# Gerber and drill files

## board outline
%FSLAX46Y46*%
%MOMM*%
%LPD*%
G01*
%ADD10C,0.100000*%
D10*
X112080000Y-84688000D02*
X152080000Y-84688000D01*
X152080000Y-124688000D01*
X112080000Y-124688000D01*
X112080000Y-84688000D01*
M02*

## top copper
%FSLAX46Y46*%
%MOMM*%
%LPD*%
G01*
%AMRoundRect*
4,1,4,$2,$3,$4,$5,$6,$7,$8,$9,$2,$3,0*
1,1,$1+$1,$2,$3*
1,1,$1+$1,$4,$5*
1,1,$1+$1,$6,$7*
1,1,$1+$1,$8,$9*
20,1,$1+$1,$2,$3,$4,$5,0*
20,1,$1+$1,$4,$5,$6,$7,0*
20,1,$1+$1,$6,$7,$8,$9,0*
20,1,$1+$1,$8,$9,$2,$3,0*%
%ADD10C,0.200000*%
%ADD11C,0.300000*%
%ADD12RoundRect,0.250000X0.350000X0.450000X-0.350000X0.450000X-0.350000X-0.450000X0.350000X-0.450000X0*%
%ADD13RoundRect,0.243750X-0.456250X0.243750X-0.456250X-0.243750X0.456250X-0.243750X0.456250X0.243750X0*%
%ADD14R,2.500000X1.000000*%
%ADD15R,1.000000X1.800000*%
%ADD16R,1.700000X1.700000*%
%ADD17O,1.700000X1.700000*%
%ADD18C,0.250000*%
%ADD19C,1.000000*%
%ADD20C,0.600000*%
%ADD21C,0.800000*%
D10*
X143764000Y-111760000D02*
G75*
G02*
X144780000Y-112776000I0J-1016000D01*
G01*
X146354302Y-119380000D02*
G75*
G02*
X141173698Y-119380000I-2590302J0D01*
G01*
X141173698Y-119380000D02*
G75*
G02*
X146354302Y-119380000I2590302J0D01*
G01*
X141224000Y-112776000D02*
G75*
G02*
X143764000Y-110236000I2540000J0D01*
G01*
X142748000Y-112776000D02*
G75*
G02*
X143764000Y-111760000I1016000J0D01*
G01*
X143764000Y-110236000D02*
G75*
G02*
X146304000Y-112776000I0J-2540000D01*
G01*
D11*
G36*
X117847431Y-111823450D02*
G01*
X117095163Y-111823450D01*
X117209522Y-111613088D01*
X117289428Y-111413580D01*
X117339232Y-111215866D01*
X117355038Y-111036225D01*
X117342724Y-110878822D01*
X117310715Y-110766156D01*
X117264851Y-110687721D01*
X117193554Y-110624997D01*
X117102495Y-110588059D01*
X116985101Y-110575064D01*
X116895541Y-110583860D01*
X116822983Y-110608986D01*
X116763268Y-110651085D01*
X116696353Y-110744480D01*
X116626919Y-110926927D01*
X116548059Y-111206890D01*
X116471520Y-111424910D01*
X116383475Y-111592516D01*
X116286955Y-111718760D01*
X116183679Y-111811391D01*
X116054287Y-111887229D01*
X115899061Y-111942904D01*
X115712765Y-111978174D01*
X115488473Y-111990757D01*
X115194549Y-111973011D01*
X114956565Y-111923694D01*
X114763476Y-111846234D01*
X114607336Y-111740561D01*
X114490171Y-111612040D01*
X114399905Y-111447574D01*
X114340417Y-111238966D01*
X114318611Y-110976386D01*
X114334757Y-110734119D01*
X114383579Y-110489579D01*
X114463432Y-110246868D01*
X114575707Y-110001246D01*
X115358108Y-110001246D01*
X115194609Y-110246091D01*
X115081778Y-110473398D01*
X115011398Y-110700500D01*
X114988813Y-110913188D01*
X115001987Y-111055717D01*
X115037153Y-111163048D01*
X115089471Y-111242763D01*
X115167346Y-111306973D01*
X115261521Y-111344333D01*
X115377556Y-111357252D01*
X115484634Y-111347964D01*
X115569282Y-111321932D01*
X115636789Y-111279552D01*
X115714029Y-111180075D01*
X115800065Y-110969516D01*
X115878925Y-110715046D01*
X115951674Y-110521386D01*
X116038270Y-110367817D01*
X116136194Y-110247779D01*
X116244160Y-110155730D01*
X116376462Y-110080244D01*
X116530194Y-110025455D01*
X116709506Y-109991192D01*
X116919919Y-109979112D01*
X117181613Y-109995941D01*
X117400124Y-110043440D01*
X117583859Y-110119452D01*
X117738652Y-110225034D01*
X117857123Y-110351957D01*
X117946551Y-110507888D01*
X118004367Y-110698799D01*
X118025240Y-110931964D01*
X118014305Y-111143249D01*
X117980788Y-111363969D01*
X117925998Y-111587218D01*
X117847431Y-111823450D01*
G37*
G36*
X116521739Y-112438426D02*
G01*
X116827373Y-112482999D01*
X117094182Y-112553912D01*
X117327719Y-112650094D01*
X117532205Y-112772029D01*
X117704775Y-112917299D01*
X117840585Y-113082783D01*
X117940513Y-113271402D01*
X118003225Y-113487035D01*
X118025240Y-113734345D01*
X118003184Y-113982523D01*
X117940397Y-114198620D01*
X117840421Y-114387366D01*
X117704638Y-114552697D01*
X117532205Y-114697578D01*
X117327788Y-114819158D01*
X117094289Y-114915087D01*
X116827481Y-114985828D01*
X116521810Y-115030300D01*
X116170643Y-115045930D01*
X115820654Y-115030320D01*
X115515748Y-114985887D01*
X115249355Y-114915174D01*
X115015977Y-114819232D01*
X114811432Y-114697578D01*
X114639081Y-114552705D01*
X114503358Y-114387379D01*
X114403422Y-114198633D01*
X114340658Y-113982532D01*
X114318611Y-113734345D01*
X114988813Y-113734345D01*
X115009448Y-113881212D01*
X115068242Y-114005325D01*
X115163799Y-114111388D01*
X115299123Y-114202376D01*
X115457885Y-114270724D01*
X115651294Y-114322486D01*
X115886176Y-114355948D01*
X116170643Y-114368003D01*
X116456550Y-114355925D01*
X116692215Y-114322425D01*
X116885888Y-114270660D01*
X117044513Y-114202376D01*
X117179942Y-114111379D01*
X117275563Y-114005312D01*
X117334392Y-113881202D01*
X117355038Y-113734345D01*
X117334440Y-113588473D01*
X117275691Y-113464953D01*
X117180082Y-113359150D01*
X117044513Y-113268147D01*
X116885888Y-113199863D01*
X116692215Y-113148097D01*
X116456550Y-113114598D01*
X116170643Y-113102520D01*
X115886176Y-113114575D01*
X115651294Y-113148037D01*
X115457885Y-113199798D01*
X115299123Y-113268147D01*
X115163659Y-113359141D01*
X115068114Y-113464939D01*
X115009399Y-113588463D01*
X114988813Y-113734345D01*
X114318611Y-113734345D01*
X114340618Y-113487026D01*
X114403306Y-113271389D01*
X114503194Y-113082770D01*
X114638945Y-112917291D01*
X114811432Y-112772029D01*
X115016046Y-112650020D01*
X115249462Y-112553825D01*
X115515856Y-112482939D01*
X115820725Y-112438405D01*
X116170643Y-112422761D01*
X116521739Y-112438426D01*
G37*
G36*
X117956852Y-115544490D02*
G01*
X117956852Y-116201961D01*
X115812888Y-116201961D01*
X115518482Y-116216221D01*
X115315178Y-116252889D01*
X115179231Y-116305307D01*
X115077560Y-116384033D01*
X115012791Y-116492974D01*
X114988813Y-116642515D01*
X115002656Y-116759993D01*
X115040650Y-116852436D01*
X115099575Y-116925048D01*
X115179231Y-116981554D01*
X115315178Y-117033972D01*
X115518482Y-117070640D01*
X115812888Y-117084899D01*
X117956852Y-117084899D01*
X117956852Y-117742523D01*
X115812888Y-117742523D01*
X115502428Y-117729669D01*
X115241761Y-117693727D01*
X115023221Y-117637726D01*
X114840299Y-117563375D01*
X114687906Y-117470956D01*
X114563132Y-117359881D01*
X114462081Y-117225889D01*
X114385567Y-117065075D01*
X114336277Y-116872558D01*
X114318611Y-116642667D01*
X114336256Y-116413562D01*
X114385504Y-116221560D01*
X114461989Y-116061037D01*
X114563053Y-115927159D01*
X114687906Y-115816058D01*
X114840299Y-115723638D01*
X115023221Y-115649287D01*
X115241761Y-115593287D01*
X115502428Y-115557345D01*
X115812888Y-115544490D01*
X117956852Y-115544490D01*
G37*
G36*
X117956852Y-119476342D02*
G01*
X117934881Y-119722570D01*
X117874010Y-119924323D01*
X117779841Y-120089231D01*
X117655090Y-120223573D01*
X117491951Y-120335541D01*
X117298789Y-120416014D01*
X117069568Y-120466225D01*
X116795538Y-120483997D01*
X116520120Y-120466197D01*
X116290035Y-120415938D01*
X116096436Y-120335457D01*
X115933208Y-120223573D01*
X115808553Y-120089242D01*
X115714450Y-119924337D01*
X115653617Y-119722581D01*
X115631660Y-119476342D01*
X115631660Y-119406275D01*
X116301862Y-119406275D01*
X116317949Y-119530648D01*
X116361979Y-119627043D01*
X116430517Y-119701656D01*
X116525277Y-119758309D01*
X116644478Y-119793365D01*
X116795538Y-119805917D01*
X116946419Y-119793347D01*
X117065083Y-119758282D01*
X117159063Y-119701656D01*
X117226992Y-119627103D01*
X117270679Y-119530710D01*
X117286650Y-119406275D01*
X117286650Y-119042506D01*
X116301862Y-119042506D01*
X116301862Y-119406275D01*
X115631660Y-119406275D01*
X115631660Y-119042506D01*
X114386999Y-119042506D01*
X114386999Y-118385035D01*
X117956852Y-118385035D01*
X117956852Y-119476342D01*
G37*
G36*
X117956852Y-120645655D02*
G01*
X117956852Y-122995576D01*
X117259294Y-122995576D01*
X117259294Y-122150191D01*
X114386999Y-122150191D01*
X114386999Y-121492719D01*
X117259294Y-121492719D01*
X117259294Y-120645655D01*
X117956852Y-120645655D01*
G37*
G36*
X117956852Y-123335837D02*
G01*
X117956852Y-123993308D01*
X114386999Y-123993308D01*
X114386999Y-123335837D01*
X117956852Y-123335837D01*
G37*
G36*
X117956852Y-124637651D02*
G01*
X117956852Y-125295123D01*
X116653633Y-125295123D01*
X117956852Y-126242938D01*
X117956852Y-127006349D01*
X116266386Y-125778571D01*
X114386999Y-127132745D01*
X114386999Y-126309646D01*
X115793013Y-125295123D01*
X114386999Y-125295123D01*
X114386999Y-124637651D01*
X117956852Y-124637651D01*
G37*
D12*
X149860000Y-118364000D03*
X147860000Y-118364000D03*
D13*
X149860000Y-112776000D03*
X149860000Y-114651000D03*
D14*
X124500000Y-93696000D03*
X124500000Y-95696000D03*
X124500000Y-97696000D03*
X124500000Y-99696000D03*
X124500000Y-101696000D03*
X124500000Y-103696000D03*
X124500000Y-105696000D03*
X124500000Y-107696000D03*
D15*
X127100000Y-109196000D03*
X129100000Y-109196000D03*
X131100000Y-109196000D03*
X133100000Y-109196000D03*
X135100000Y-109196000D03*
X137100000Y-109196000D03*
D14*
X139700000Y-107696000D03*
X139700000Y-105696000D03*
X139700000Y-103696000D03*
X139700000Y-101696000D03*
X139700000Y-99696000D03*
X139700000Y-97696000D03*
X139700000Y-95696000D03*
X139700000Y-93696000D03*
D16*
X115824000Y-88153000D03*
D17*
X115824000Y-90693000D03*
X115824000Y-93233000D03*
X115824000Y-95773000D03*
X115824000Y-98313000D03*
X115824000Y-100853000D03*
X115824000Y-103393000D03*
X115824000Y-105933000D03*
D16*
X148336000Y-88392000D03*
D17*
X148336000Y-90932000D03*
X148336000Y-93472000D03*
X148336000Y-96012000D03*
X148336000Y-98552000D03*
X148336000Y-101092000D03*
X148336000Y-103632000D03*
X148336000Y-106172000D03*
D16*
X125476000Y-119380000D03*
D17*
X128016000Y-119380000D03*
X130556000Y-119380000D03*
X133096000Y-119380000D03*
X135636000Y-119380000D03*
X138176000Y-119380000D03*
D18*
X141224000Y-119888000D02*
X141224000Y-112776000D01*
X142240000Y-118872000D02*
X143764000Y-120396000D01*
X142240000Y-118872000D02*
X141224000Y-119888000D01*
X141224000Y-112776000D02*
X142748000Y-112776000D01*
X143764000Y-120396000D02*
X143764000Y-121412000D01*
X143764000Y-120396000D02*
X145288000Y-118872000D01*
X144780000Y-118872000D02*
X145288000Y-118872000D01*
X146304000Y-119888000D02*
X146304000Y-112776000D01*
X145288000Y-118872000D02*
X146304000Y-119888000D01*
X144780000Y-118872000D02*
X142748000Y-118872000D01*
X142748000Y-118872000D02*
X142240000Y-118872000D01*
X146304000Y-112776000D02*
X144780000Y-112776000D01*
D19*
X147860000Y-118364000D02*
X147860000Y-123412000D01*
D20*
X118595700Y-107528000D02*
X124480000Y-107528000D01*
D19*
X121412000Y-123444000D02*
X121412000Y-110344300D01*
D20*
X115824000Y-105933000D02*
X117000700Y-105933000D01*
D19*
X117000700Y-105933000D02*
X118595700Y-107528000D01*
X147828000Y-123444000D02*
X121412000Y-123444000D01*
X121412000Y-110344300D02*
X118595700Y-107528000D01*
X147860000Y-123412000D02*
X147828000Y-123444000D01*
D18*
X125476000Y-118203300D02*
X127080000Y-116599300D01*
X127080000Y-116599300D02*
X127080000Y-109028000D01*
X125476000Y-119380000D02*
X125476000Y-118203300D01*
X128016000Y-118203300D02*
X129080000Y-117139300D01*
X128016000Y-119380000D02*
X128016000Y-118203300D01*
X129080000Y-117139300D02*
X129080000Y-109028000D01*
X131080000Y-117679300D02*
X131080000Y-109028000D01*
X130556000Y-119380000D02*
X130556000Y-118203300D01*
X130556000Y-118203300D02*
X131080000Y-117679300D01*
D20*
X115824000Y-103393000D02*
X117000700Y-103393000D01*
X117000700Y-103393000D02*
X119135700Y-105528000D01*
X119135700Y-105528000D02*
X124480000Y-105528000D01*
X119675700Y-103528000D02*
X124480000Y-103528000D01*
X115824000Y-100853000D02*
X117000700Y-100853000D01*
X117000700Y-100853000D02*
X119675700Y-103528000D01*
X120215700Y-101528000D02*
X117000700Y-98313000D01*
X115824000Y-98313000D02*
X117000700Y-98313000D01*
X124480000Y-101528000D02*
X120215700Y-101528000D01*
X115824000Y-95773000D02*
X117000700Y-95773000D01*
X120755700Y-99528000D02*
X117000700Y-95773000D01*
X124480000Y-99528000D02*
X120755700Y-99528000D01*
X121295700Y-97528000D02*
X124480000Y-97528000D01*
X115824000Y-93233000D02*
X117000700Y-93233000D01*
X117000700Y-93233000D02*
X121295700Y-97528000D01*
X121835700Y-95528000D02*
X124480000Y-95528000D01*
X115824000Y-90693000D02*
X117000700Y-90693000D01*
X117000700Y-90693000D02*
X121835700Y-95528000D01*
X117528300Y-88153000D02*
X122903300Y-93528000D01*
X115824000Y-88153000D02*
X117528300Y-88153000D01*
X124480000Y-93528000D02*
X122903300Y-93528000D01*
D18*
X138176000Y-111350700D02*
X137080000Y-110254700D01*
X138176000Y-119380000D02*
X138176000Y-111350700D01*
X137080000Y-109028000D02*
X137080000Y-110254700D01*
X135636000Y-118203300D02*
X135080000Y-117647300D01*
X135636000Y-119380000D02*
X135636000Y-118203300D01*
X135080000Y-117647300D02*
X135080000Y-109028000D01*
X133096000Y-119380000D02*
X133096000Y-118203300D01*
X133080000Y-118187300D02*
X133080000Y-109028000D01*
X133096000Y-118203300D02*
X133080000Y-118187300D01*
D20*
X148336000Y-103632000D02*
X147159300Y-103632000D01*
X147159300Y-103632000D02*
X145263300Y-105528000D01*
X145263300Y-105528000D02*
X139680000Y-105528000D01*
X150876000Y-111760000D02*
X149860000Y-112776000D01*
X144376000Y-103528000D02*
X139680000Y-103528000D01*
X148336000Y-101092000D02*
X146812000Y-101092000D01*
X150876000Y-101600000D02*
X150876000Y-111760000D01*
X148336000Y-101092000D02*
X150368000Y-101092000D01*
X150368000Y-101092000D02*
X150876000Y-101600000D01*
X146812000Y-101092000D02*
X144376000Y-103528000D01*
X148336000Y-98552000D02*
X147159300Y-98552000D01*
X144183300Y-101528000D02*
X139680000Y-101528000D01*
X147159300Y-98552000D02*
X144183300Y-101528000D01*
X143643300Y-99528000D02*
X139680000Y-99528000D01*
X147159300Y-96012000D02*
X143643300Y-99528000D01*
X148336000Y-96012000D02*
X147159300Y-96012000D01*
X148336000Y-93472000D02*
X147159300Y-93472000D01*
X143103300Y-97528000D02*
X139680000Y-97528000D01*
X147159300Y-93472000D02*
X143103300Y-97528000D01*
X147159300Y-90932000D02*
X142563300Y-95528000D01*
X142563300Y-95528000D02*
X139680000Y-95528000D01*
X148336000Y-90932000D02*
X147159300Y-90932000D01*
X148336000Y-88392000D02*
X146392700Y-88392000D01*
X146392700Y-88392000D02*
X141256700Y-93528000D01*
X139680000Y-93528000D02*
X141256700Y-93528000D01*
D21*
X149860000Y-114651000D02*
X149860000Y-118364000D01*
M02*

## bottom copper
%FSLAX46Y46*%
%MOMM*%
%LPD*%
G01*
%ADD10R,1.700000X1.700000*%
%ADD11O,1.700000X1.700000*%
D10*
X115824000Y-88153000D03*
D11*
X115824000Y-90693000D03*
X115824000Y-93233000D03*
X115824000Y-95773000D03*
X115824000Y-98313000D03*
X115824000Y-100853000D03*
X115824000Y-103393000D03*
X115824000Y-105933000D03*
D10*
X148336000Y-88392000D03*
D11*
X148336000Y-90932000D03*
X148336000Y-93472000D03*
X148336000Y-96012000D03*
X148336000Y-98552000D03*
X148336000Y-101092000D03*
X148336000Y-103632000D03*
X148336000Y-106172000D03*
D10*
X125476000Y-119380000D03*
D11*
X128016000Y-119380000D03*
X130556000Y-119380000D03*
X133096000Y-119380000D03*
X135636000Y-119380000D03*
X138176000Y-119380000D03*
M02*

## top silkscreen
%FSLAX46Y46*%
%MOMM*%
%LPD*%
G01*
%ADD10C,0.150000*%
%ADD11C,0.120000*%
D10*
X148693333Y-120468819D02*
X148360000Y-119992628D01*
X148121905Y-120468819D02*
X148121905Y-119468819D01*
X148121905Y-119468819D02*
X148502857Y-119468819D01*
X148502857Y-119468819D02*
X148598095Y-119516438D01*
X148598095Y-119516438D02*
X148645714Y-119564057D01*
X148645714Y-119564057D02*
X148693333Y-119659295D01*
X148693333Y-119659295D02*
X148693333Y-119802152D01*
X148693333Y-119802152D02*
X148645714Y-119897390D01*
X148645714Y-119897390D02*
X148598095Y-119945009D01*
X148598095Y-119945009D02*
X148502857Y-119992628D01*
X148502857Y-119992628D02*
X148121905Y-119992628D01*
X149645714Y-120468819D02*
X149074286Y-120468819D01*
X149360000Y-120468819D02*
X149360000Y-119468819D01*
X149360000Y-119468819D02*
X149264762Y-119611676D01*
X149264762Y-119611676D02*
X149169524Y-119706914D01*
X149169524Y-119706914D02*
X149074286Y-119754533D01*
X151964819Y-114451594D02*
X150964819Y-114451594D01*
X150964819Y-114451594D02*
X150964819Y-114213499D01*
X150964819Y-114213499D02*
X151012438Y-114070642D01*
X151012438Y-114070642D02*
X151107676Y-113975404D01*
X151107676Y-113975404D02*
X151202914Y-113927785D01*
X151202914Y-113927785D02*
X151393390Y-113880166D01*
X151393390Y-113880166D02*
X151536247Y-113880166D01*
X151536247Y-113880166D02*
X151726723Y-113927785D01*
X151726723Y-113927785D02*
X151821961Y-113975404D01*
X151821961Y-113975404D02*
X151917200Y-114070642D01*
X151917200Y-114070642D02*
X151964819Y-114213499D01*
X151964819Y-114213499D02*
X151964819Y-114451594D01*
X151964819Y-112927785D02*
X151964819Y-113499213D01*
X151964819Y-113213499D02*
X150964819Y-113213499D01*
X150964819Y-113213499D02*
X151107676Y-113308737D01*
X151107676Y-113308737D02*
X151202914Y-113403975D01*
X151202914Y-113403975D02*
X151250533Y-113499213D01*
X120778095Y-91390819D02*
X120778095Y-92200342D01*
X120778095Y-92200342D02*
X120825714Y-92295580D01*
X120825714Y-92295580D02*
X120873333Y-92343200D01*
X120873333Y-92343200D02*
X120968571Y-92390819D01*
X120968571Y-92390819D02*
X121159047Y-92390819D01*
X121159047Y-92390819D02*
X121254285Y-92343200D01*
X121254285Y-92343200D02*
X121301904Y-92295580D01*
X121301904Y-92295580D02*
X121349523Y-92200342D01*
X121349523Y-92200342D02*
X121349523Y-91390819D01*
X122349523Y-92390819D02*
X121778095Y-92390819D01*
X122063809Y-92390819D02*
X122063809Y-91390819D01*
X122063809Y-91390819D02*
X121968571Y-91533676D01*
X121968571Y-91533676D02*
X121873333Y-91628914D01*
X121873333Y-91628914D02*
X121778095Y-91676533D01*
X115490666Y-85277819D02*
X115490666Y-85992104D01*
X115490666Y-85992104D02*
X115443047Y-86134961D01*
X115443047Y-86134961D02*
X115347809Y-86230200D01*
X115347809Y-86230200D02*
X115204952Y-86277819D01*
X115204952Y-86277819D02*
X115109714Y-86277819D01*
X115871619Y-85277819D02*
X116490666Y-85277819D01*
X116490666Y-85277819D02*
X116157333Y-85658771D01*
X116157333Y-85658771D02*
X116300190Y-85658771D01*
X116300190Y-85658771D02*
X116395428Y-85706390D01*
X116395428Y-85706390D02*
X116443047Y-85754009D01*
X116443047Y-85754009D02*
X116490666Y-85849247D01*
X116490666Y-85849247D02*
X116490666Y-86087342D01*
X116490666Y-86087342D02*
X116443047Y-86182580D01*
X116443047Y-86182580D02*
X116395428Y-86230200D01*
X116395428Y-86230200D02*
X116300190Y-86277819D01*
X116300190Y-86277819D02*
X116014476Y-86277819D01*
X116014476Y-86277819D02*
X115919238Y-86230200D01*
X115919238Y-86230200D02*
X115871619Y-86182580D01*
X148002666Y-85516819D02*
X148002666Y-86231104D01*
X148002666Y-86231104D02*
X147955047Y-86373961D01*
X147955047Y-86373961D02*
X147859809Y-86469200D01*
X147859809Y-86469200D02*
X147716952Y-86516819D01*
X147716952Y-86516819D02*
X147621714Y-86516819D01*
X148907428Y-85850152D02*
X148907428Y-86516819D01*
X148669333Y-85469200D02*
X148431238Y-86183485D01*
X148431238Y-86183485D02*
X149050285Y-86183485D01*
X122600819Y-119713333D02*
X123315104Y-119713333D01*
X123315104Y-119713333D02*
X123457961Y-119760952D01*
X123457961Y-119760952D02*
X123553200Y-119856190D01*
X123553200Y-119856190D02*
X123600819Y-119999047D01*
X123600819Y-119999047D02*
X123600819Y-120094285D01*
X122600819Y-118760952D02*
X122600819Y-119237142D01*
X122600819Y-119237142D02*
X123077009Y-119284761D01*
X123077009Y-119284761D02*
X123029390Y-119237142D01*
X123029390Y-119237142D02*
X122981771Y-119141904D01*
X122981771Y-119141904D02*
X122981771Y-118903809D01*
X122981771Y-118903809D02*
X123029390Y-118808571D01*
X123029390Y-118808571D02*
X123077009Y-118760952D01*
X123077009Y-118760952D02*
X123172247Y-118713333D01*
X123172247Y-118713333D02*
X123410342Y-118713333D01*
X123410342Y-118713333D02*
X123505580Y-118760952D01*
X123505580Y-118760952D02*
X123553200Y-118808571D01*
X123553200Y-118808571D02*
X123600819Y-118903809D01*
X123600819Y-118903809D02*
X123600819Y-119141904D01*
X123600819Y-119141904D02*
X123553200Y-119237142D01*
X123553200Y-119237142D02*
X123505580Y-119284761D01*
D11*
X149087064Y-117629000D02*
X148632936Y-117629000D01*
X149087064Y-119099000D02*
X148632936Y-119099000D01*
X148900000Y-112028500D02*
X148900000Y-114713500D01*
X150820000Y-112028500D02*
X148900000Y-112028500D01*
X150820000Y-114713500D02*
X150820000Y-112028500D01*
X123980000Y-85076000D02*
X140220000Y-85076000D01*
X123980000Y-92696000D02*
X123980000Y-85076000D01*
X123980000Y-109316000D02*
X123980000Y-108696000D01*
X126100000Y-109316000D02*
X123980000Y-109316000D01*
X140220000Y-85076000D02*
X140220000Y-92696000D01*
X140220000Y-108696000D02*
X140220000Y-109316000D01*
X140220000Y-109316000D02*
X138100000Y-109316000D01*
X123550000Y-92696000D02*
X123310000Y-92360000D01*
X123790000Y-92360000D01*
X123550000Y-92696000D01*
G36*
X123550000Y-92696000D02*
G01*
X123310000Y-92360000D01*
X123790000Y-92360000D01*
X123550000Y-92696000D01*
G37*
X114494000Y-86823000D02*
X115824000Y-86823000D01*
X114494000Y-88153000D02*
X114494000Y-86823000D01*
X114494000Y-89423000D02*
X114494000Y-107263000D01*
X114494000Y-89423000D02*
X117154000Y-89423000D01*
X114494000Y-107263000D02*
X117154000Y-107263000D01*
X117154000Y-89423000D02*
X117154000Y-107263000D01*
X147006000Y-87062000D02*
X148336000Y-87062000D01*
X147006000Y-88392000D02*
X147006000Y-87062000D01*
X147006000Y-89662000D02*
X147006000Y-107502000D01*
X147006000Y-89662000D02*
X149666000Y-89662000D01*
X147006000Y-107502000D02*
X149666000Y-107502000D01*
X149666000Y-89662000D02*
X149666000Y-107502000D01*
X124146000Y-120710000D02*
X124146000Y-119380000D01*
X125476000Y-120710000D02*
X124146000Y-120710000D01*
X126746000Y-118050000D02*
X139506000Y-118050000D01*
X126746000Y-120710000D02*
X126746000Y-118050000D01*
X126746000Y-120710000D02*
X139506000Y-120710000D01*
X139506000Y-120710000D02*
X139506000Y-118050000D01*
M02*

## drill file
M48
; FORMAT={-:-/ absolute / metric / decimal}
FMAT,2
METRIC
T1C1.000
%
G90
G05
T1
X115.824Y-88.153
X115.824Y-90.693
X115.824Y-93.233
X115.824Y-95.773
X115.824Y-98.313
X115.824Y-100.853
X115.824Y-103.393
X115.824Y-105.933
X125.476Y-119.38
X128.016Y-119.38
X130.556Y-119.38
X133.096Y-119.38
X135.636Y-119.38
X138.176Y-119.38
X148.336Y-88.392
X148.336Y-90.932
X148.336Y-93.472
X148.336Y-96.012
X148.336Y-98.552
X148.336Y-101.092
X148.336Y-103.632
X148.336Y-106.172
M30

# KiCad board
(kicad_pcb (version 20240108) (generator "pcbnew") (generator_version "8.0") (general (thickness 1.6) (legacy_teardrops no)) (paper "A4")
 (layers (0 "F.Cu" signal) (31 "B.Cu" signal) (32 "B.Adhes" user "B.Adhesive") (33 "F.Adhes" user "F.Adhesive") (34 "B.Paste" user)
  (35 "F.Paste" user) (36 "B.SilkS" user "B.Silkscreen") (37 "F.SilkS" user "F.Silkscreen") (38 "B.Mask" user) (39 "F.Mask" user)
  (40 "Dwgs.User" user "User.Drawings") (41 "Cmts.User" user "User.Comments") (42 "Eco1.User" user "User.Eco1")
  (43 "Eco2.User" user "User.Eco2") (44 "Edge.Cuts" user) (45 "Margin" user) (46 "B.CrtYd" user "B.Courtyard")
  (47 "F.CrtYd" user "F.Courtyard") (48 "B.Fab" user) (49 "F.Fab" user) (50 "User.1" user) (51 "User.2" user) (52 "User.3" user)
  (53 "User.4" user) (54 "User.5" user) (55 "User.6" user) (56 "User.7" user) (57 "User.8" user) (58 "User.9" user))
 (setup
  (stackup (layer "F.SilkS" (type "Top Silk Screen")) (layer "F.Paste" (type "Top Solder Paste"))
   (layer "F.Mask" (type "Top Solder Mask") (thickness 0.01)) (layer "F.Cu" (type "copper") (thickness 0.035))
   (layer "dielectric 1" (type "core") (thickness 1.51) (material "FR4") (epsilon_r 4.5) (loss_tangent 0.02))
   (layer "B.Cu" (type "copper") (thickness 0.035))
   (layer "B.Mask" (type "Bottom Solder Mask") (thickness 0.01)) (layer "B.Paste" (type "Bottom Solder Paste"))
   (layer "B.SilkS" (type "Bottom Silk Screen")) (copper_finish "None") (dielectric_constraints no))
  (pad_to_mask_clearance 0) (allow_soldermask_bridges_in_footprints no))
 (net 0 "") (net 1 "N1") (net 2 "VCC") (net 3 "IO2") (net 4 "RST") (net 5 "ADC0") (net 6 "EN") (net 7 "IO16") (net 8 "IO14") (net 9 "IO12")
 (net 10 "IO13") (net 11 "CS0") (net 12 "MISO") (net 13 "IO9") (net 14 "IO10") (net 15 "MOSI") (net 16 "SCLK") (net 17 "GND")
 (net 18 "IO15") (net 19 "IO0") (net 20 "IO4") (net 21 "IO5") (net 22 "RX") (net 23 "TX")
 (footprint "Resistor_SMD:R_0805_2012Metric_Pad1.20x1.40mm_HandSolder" (layer "F.Cu") (at 148.86 118.364 180)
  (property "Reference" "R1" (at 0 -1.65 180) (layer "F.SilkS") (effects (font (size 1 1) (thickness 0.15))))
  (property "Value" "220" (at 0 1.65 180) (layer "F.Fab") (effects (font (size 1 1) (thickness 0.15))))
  (fp_line (start -0.227064 0.735) (end 0.227064 0.735) (stroke (width 0.12) (type solid)) (layer "F.SilkS"))
  (fp_line (start -0.227064 -0.735) (end 0.227064 -0.735) (stroke (width 0.12) (type solid)) (layer "F.SilkS"))
  (pad "1" smd roundrect (at -1 0 180) (size 1.2 1.4) (layers "F.Cu" "F.Paste" "F.Mask") (roundrect_rratio 0.208333) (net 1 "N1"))
  (pad "2" smd roundrect (at 1 0 180) (size 1.2 1.4) (layers "F.Cu" "F.Paste" "F.Mask") (roundrect_rratio 0.208333) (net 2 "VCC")))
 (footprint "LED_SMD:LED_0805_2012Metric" (layer "F.Cu") (at 149.86 113.7135 -90)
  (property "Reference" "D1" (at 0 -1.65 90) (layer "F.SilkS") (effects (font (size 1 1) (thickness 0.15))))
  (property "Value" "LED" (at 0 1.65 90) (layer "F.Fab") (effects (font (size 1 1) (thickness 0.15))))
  (fp_line (start -1.685 0.96) (end 1 0.96) (stroke (width 0.12) (type solid)) (layer "F.SilkS"))
  (fp_line (start -1.685 -0.96) (end -1.685 0.96) (stroke (width 0.12) (type solid)) (layer "F.SilkS"))
  (fp_line (start 1 -0.96) (end -1.685 -0.96) (stroke (width 0.12) (type solid)) (layer "F.SilkS"))
  (pad "1" smd roundrect (at -0.9375 0 270) (size 0.975 1.4) (layers "F.Cu" "F.Paste" "F.Mask") (roundrect_rratio 0.25) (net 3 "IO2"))
  (pad "2" smd roundrect (at 0.9375 0 270) (size 0.975 1.4) (layers "F.Cu" "F.Paste" "F.Mask") (roundrect_rratio 0.25) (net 1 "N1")))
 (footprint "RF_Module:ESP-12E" (layer "F.Cu") (at 132.1 97.196)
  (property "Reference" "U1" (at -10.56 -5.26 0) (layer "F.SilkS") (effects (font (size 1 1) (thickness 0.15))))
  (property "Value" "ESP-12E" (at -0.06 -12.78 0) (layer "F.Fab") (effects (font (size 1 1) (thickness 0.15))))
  (fp_line (start -8.12 -12.12) (end 8.12 -12.12) (stroke (width 0.12) (type solid)) (layer "F.SilkS"))
  (fp_line (start -8.12 -4.5) (end -8.12 -12.12) (stroke (width 0.12) (type solid)) (layer "F.SilkS"))
  (fp_line (start -8.12 12.12) (end -8.12 11.5) (stroke (width 0.12) (type solid)) (layer "F.SilkS"))
  (fp_line (start -6 12.12) (end -8.12 12.12) (stroke (width 0.12) (type solid)) (layer "F.SilkS"))
  (fp_line (start 8.12 -12.12) (end 8.12 -4.5) (stroke (width 0.12) (type solid)) (layer "F.SilkS"))
  (fp_line (start 8.12 11.5) (end 8.12 12.12) (stroke (width 0.12) (type solid)) (layer "F.SilkS"))
  (fp_line (start 8.12 12.12) (end 6 12.12) (stroke (width 0.12) (type solid)) (layer "F.SilkS"))
  (fp_poly
   (pts (xy -8.55 -4.5) (xy -8.79 -4.836) (xy -8.31 -4.836) (xy -8.55 -4.5)) (stroke (width 0.12) (type solid)) (fill solid)
   (layer "F.SilkS"))
  (pad "1" smd rect (at -7.6 -3.5) (size 2.5 1) (layers "F.Cu" "F.Paste" "F.Mask") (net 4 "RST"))
  (pad "2" smd rect (at -7.6 -1.5) (size 2.5 1) (layers "F.Cu" "F.Paste" "F.Mask") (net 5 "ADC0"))
  (pad "3" smd rect (at -7.6 0.5) (size 2.5 1) (layers "F.Cu" "F.Paste" "F.Mask") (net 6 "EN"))
  (pad "4" smd rect (at -7.6 2.5) (size 2.5 1) (layers "F.Cu" "F.Paste" "F.Mask") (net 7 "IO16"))
  (pad "5" smd rect (at -7.6 4.5) (size 2.5 1) (layers "F.Cu" "F.Paste" "F.Mask") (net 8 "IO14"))
  (pad "6" smd rect (at -7.6 6.5) (size 2.5 1) (layers "F.Cu" "F.Paste" "F.Mask") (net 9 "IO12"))
  (pad "7" smd rect (at -7.6 8.5) (size 2.5 1) (layers "F.Cu" "F.Paste" "F.Mask") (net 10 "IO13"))
  (pad "8" smd rect (at -7.6 10.5) (size 2.5 1) (layers "F.Cu" "F.Paste" "F.Mask") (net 2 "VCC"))
  (pad "9" smd rect (at -5 12) (size 1 1.8) (layers "F.Cu" "F.Paste" "F.Mask") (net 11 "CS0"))
  (pad "10" smd rect (at -3 12) (size 1 1.8) (layers "F.Cu" "F.Paste" "F.Mask") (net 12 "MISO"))
  (pad "11" smd rect (at -1 12) (size 1 1.8) (layers "F.Cu" "F.Paste" "F.Mask") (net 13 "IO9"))
  (pad "12" smd rect (at 1 12) (size 1 1.8) (layers "F.Cu" "F.Paste" "F.Mask") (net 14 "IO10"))
  (pad "13" smd rect (at 3 12) (size 1 1.8) (layers "F.Cu" "F.Paste" "F.Mask") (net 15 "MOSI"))
  (pad "14" smd rect (at 5 12) (size 1 1.8) (layers "F.Cu" "F.Paste" "F.Mask") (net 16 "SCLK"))
  (pad "15" smd rect (at 7.6 10.5) (size 2.5 1) (layers "F.Cu" "F.Paste" "F.Mask") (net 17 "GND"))
  (pad "16" smd rect (at 7.6 8.5) (size 2.5 1) (layers "F.Cu" "F.Paste" "F.Mask") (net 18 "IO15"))
  (pad "17" smd rect (at 7.6 6.5) (size 2.5 1) (layers "F.Cu" "F.Paste" "F.Mask") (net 3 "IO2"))
  (pad "18" smd rect (at 7.6 4.5) (size 2.5 1) (layers "F.Cu" "F.Paste" "F.Mask") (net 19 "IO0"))
  (pad "19" smd rect (at 7.6 2.5) (size 2.5 1) (layers "F.Cu" "F.Paste" "F.Mask") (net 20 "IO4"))
  (pad "20" smd rect (at 7.6 0.5) (size 2.5 1) (layers "F.Cu" "F.Paste" "F.Mask") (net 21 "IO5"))
  (pad "21" smd rect (at 7.6 -1.5) (size 2.5 1) (layers "F.Cu" "F.Paste" "F.Mask") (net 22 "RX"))
  (pad "22" smd rect (at 7.6 -3.5) (size 2.5 1) (layers "F.Cu" "F.Paste" "F.Mask") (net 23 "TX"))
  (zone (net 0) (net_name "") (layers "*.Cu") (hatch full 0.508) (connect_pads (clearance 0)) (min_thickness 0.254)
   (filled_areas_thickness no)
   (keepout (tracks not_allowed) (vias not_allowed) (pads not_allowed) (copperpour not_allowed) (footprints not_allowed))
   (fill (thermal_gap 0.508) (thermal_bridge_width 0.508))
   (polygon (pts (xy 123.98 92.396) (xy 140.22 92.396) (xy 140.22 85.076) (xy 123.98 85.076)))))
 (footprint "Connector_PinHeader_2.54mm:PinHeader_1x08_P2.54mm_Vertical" (layer "F.Cu") (at 115.824 88.153)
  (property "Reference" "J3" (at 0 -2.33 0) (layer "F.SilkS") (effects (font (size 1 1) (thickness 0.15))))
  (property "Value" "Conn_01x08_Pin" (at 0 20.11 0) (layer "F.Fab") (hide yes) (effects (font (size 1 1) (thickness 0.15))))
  (fp_line (start -1.33 -1.33) (end 0 -1.33) (stroke (width 0.12) (type solid)) (layer "F.SilkS"))
  (fp_line (start -1.33 0) (end -1.33 -1.33) (stroke (width 0.12) (type solid)) (layer "F.SilkS"))
  (fp_line (start -1.33 1.27) (end -1.33 19.11) (stroke (width 0.12) (type solid)) (layer "F.SilkS"))
  (fp_line (start -1.33 1.27) (end 1.33 1.27) (stroke (width 0.12) (type solid)) (layer "F.SilkS"))
  (fp_line (start -1.33 19.11) (end 1.33 19.11) (stroke (width 0.12) (type solid)) (layer "F.SilkS"))
  (fp_line (start 1.33 1.27) (end 1.33 19.11) (stroke (width 0.12) (type solid)) (layer "F.SilkS"))
  (pad "1" thru_hole rect (at 0 0) (size 1.7 1.7) (drill 1) (layers "*.Cu" "*.Mask") (remove_unused_layers no) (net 4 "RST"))
  (pad "2" thru_hole oval (at 0 2.54) (size 1.7 1.7) (drill 1) (layers "*.Cu" "*.Mask") (remove_unused_layers no) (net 5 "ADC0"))
  (pad "3" thru_hole oval (at 0 5.08) (size 1.7 1.7) (drill 1) (layers "*.Cu" "*.Mask") (remove_unused_layers no) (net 6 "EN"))
  (pad "4" thru_hole oval (at 0 7.62) (size 1.7 1.7) (drill 1) (layers "*.Cu" "*.Mask") (remove_unused_layers no) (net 7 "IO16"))
  (pad "5" thru_hole oval (at 0 10.16) (size 1.7 1.7) (drill 1) (layers "*.Cu" "*.Mask") (remove_unused_layers no) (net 8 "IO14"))
  (pad "6" thru_hole oval (at 0 12.7) (size 1.7 1.7) (drill 1) (layers "*.Cu" "*.Mask") (remove_unused_layers no) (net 9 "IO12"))
  (pad "7" thru_hole oval (at 0 15.24) (size 1.7 1.7) (drill 1) (layers "*.Cu" "*.Mask") (remove_unused_layers no) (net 10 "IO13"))
  (pad "8" thru_hole oval (at 0 17.78) (size 1.7 1.7) (drill 1) (layers "*.Cu" "*.Mask") (remove_unused_layers no) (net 2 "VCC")))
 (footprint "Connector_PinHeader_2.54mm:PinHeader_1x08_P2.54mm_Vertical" (layer "F.Cu") (at 148.336 88.392)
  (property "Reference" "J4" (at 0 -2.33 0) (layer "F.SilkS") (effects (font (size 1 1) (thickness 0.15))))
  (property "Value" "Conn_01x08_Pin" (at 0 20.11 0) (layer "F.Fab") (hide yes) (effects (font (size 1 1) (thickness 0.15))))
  (fp_line (start -1.33 -1.33) (end 0 -1.33) (stroke (width 0.12) (type solid)) (layer "F.SilkS"))
  (fp_line (start -1.33 0) (end -1.33 -1.33) (stroke (width 0.12) (type solid)) (layer "F.SilkS"))
  (fp_line (start -1.33 1.27) (end -1.33 19.11) (stroke (width 0.12) (type solid)) (layer "F.SilkS"))
  (fp_line (start -1.33 1.27) (end 1.33 1.27) (stroke (width 0.12) (type solid)) (layer "F.SilkS"))
  (fp_line (start -1.33 19.11) (end 1.33 19.11) (stroke (width 0.12) (type solid)) (layer "F.SilkS"))
  (fp_line (start 1.33 1.27) (end 1.33 19.11) (stroke (width 0.12) (type solid)) (layer "F.SilkS"))
  (pad "1" thru_hole rect (at 0 0) (size 1.7 1.7) (drill 1) (layers "*.Cu" "*.Mask") (remove_unused_layers no) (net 23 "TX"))
  (pad "2" thru_hole oval (at 0 2.54) (size 1.7 1.7) (drill 1) (layers "*.Cu" "*.Mask") (remove_unused_layers no) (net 22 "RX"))
  (pad "3" thru_hole oval (at 0 5.08) (size 1.7 1.7) (drill 1) (layers "*.Cu" "*.Mask") (remove_unused_layers no) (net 21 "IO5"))
  (pad "4" thru_hole oval (at 0 7.62) (size 1.7 1.7) (drill 1) (layers "*.Cu" "*.Mask") (remove_unused_layers no) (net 20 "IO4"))
  (pad "5" thru_hole oval (at 0 10.16) (size 1.7 1.7) (drill 1) (layers "*.Cu" "*.Mask") (remove_unused_layers no) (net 19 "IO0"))
  (pad "6" thru_hole oval (at 0 12.7) (size 1.7 1.7) (drill 1) (layers "*.Cu" "*.Mask") (remove_unused_layers no) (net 3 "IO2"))
  (pad "7" thru_hole oval (at 0 15.24) (size 1.7 1.7) (drill 1) (layers "*.Cu" "*.Mask") (remove_unused_layers no) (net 18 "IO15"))
  (pad "8" thru_hole oval (at 0 17.78) (size 1.7 1.7) (drill 1) (layers "*.Cu" "*.Mask") (remove_unused_layers no) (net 17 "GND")))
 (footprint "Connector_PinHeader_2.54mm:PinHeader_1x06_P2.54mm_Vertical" (layer "F.Cu") (at 125.476 119.38 90)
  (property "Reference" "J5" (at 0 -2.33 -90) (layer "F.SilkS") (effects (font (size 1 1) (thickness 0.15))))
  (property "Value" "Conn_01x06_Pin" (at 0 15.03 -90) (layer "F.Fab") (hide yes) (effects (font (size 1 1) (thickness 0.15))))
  (fp_line (start -1.33 -1.33) (end 0 -1.33) (stroke (width 0.12) (type solid)) (layer "F.SilkS"))
  (fp_line (start -1.33 0) (end -1.33 -1.33) (stroke (width 0.12) (type solid)) (layer "F.SilkS"))
  (fp_line (start 1.33 1.27) (end 1.33 14.03) (stroke (width 0.12) (type solid)) (layer "F.SilkS"))
  (fp_line (start -1.33 1.27) (end 1.33 1.27) (stroke (width 0.12) (type solid)) (layer "F.SilkS"))
  (fp_line (start -1.33 1.27) (end -1.33 14.03) (stroke (width 0.12) (type solid)) (layer "F.SilkS"))
  (fp_line (start -1.33 14.03) (end 1.33 14.03) (stroke (width 0.12) (type solid)) (layer "F.SilkS"))
  (pad "1" thru_hole rect (at 0 0 90) (size 1.7 1.7) (drill 1) (layers "*.Cu" "*.Mask") (remove_unused_layers no) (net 11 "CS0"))
  (pad "2" thru_hole oval (at 0 2.54 90) (size 1.7 1.7) (drill 1) (layers "*.Cu" "*.Mask") (remove_unused_layers no) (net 12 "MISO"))
  (pad "3" thru_hole oval (at 0 5.08 90) (size 1.7 1.7) (drill 1) (layers "*.Cu" "*.Mask") (remove_unused_layers no) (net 13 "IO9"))
  (pad "4" thru_hole oval (at 0 7.62 90) (size 1.7 1.7) (drill 1) (layers "*.Cu" "*.Mask") (remove_unused_layers no) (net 14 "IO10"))
  (pad "5" thru_hole oval (at 0 10.16 90) (size 1.7 1.7) (drill 1) (layers "*.Cu" "*.Mask") (remove_unused_layers no) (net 15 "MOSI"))
  (pad "6" thru_hole oval (at 0 12.7 90) (size 1.7 1.7) (drill 1) (layers "*.Cu" "*.Mask") (remove_unused_layers no) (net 16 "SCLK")))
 (gr_arc (start 143.764 111.76) (mid 144.48242 112.05758) (end 144.78 112.776) (stroke (width 0.2) (type default)) (layer "F.Cu"))
 (gr_circle (center 143.764 119.38) (end 143.256 121.92) (stroke (width 0.2) (type default)) (fill none) (layer "F.Cu"))
 (gr_arc (start 141.224 112.776) (mid 141.967949 110.979949) (end 143.764 110.236) (stroke (width 0.2) (type default)) (layer "F.Cu"))
 (gr_arc (start 142.748 112.776) (mid 143.04558 112.05758) (end 143.764 111.76) (stroke (width 0.2) (type default)) (layer "F.Cu"))
 (gr_arc (start 143.764 110.236) (mid 145.560051 110.979949) (end 146.304 112.776) (stroke (width 0.2) (type default)) (layer "F.Cu"))
 (gr_rect (start 112.08 84.688) (end 152.08 124.688) (stroke (width 0.1) (type default)) (fill none) (layer "Edge.Cuts"))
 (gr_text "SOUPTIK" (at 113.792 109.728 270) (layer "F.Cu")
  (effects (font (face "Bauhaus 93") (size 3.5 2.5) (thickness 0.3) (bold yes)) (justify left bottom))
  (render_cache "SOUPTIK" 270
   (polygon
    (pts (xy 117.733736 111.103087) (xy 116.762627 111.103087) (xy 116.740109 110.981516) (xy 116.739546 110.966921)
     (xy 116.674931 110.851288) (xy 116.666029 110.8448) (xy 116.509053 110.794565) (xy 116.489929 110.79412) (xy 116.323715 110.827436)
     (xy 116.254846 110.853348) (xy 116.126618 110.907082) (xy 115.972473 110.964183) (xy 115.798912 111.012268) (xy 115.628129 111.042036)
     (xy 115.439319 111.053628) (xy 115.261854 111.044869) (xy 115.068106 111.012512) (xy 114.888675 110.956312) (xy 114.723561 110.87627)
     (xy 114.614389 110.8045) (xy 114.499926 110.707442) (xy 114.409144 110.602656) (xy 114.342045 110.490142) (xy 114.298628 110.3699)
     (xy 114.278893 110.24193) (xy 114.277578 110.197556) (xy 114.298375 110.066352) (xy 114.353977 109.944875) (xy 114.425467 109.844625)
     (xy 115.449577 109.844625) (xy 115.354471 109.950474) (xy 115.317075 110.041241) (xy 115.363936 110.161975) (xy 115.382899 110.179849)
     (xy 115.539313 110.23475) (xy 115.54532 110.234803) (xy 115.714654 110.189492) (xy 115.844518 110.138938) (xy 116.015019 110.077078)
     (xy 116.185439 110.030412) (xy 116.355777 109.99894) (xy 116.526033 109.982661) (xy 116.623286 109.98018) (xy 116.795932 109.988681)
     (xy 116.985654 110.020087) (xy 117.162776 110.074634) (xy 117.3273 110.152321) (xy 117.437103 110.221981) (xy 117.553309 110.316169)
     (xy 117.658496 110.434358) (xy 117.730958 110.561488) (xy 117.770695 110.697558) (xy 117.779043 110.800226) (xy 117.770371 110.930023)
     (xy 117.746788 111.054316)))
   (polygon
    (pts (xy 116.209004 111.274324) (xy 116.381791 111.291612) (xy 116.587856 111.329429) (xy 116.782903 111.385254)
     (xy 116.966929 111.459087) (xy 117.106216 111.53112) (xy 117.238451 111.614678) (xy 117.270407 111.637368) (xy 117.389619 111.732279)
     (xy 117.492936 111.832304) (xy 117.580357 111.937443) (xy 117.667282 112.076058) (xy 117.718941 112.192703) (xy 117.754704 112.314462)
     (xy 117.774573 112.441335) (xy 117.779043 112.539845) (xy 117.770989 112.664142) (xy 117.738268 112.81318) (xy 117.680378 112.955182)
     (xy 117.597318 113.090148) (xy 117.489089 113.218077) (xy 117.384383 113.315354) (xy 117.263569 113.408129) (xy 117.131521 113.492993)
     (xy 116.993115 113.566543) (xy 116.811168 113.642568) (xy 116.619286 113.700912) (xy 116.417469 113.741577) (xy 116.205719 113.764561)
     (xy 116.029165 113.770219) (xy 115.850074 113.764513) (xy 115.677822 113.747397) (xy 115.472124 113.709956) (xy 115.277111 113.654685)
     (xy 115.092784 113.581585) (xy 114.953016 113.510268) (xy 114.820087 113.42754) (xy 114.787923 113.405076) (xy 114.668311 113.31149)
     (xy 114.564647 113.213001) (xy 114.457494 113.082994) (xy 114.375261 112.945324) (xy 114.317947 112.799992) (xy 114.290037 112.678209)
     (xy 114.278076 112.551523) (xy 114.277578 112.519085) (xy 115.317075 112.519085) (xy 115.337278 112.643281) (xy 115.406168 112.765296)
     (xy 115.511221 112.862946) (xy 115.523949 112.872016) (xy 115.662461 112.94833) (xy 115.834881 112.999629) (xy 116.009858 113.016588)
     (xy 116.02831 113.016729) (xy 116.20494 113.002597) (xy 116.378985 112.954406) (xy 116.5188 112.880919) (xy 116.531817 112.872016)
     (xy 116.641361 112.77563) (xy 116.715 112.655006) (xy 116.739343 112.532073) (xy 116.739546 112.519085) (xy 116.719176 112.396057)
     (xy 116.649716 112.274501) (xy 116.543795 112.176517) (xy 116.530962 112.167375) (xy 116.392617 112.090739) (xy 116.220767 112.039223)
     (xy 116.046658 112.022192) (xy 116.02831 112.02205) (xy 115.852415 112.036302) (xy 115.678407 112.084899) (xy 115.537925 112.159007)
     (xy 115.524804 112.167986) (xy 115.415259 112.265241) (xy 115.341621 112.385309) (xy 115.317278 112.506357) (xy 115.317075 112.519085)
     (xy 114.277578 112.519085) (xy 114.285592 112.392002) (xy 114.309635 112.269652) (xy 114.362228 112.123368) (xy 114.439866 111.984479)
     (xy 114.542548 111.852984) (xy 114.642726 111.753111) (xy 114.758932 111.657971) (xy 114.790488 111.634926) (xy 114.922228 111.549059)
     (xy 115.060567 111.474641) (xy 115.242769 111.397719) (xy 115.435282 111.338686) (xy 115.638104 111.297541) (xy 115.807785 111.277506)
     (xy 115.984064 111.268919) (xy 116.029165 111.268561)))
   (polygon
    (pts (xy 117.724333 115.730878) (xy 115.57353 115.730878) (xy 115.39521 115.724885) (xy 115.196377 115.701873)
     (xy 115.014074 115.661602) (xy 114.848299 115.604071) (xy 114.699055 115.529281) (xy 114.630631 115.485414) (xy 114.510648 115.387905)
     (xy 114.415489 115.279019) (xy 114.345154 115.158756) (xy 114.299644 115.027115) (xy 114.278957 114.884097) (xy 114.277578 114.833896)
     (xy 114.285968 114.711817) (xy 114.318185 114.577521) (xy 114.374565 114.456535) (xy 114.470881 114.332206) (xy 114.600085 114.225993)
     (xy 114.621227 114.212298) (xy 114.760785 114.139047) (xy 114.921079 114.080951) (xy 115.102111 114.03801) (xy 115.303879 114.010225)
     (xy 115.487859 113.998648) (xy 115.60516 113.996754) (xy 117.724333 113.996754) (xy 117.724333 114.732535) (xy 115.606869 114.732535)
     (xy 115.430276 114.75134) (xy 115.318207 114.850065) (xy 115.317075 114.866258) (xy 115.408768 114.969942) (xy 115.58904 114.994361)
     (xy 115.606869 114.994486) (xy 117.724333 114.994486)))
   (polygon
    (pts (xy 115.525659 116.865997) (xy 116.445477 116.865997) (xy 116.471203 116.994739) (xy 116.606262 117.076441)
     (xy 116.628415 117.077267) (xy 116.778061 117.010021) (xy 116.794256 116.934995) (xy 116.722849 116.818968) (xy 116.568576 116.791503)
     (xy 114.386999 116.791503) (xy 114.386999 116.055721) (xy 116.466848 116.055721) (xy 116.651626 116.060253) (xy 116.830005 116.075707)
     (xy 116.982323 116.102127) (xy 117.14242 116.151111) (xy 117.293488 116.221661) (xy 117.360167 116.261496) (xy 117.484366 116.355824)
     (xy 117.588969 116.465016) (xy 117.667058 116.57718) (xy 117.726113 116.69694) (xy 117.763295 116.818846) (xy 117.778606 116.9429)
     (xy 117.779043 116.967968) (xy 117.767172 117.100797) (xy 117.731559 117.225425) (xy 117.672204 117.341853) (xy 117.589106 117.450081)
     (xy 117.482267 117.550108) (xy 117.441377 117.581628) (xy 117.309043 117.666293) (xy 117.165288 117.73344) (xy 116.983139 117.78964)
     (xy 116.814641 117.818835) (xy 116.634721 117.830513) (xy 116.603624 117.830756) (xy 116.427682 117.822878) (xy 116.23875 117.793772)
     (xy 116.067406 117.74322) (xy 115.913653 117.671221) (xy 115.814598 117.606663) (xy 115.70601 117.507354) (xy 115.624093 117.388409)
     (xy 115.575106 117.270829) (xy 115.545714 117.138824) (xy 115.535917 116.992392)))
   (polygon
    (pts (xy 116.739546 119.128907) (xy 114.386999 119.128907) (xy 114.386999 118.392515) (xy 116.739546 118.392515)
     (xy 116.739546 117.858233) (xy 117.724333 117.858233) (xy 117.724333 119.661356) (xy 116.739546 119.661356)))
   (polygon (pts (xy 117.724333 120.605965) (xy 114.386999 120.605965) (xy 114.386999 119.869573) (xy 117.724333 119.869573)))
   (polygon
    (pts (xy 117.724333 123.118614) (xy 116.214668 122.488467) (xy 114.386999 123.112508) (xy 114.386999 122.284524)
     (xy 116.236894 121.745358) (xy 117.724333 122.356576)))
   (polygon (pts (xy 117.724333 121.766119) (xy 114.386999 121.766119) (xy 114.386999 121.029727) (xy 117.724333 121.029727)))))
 (segment (start 141.224 119.888) (end 141.224 112.776) (width 0.25) (layer "F.Cu") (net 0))
 (segment (start 142.24 118.872) (end 143.764 120.396) (width 0.25) (layer "F.Cu") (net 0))
 (segment (start 142.24 118.872) (end 141.224 119.888) (width 0.25) (layer "F.Cu") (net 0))
 (segment (start 141.224 112.776) (end 142.748 112.776) (width 0.25) (layer "F.Cu") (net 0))
 (segment (start 143.764 120.396) (end 143.764 121.412) (width 0.25) (layer "F.Cu") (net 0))
 (segment (start 143.764 120.396) (end 145.288 118.872) (width 0.25) (layer "F.Cu") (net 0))
 (segment (start 144.78 118.872) (end 145.288 118.872) (width 0.25) (layer "F.Cu") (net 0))
 (segment (start 146.304 119.888) (end 146.304 112.776) (width 0.25) (layer "F.Cu") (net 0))
 (segment (start 145.288 118.872) (end 146.304 119.888) (width 0.25) (layer "F.Cu") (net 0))
 (segment (start 144.78 118.872) (end 142.748 118.872) (width 0.25) (layer "F.Cu") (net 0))
 (segment (start 142.748 118.872) (end 142.24 118.872) (width 0.25) (layer "F.Cu") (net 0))
 (segment (start 146.304 112.776) (end 144.78 112.776) (width 0.25) (layer "F.Cu") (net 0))
 (segment (start 147.86 118.364) (end 147.86 123.412) (width 1) (layer "F.Cu") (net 2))
 (segment (start 118.5957 107.528) (end 124.48 107.528) (width 0.6) (layer "F.Cu") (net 2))
 (segment (start 121.412 123.444) (end 121.412 110.3443) (width 1) (layer "F.Cu") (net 2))
 (segment (start 115.824 105.933) (end 117.0007 105.933) (width 0.6) (layer "F.Cu") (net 2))
 (segment (start 117.0007 105.933) (end 118.5957 107.528) (width 1) (layer "F.Cu") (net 2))
 (segment (start 147.828 123.444) (end 121.412 123.444) (width 1) (layer "F.Cu") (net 2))
 (segment (start 121.412 110.3443) (end 118.5957 107.528) (width 1) (layer "F.Cu") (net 2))
 (segment (start 147.86 123.412) (end 147.828 123.444) (width 1) (layer "F.Cu") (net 2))
 (segment (start 125.476 118.2033) (end 127.08 116.5993) (width 0.25) (layer "F.Cu") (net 11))
 (segment (start 127.08 116.5993) (end 127.08 109.028) (width 0.25) (layer "F.Cu") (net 11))
 (segment (start 125.476 119.38) (end 125.476 118.2033) (width 0.25) (layer "F.Cu") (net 11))
 (segment (start 128.016 118.2033) (end 129.08 117.1393) (width 0.25) (layer "F.Cu") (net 12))
 (segment (start 128.016 119.38) (end 128.016 118.2033) (width 0.25) (layer "F.Cu") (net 12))
 (segment (start 129.08 117.1393) (end 129.08 109.028) (width 0.25) (layer "F.Cu") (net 12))
 (segment (start 131.08 117.6793) (end 131.08 109.028) (width 0.25) (layer "F.Cu") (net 13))
 (segment (start 130.556 119.38) (end 130.556 118.2033) (width 0.25) (layer "F.Cu") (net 13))
 (segment (start 130.556 118.2033) (end 131.08 117.6793) (width 0.25) (layer "F.Cu") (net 13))
 (segment (start 115.824 103.393) (end 117.0007 103.393) (width 0.6) (layer "F.Cu") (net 10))
 (segment (start 117.0007 103.393) (end 119.1357 105.528) (width 0.6) (layer "F.Cu") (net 10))
 (segment (start 119.1357 105.528) (end 124.48 105.528) (width 0.6) (layer "F.Cu") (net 10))
 (segment (start 119.6757 103.528) (end 124.48 103.528) (width 0.6) (layer "F.Cu") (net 9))
 (segment (start 115.824 100.853) (end 117.0007 100.853) (width 0.6) (layer "F.Cu") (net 9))
 (segment (start 117.0007 100.853) (end 119.6757 103.528) (width 0.6) (layer "F.Cu") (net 9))
 (segment (start 120.2157 101.528) (end 117.0007 98.313) (width 0.6) (layer "F.Cu") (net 8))
 (segment (start 115.824 98.313) (end 117.0007 98.313) (width 0.6) (layer "F.Cu") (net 8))
 (segment (start 124.48 101.528) (end 120.2157 101.528) (width 0.6) (layer "F.Cu") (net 8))
 (segment (start 115.824 95.773) (end 117.0007 95.773) (width 0.6) (layer "F.Cu") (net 7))
 (segment (start 120.7557 99.528) (end 117.0007 95.773) (width 0.6) (layer "F.Cu") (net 7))
 (segment (start 124.48 99.528) (end 120.7557 99.528) (width 0.6) (layer "F.Cu") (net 7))
 (segment (start 121.2957 97.528) (end 124.48 97.528) (width 0.6) (layer "F.Cu") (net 6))
 (segment (start 115.824 93.233) (end 117.0007 93.233) (width 0.6) (layer "F.Cu") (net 6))
 (segment (start 117.0007 93.233) (end 121.2957 97.528) (width 0.6) (layer "F.Cu") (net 6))
 (segment (start 121.8357 95.528) (end 124.48 95.528) (width 0.6) (layer "F.Cu") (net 5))
 (segment (start 115.824 90.693) (end 117.0007 90.693) (width 0.6) (layer "F.Cu") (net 5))
 (segment (start 117.0007 90.693) (end 121.8357 95.528) (width 0.6) (layer "F.Cu") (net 5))
 (segment (start 117.5283 88.153) (end 122.9033 93.528) (width 0.6) (layer "F.Cu") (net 4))
 (segment (start 115.824 88.153) (end 117.5283 88.153) (width 0.6) (layer "F.Cu") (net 4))
 (segment (start 124.48 93.528) (end 122.9033 93.528) (width 0.6) (layer "F.Cu") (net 4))
 (segment (start 138.176 111.3507) (end 137.08 110.2547) (width 0.25) (layer "F.Cu") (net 16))
 (segment (start 138.176 119.38) (end 138.176 111.3507) (width 0.25) (layer "F.Cu") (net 16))
 (segment (start 137.08 109.028) (end 137.08 110.2547) (width 0.25) (layer "F.Cu") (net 16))
 (segment (start 135.636 118.2033) (end 135.08 117.6473) (width 0.25) (layer "F.Cu") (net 15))
 (segment (start 135.636 119.38) (end 135.636 118.2033) (width 0.25) (layer "F.Cu") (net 15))
 (segment (start 135.08 117.6473) (end 135.08 109.028) (width 0.25) (layer "F.Cu") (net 15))
 (segment (start 133.096 119.38) (end 133.096 118.2033) (width 0.25) (layer "F.Cu") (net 14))
 (segment (start 133.08 118.1873) (end 133.08 109.028) (width 0.25) (layer "F.Cu") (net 14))
 (segment (start 133.096 118.2033) (end 133.08 118.1873) (width 0.25) (layer "F.Cu") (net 14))
 (segment (start 148.336 103.632) (end 147.1593 103.632) (width 0.6) (layer "F.Cu") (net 18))
 (segment (start 147.1593 103.632) (end 145.2633 105.528) (width 0.6) (layer "F.Cu") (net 18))
 (segment (start 145.2633 105.528) (end 139.68 105.528) (width 0.6) (layer "F.Cu") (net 18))
 (segment (start 150.876 111.76) (end 149.86 112.776) (width 0.6) (layer "F.Cu") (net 3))
 (segment (start 144.376 103.528) (end 139.68 103.528) (width 0.6) (layer "F.Cu") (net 3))
 (segment (start 148.336 101.092) (end 146.812 101.092) (width 0.6) (layer "F.Cu") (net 3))
 (segment (start 150.876 101.6) (end 150.876 111.76) (width 0.6) (layer "F.Cu") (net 3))
 (segment (start 148.336 101.092) (end 150.368 101.092) (width 0.6) (layer "F.Cu") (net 3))
 (segment (start 150.368 101.092) (end 150.876 101.6) (width 0.6) (layer "F.Cu") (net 3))
 (segment (start 146.812 101.092) (end 144.376 103.528) (width 0.6) (layer "F.Cu") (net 3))
 (segment (start 148.336 98.552) (end 147.1593 98.552) (width 0.6) (layer "F.Cu") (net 19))
 (segment (start 144.1833 101.528) (end 139.68 101.528) (width 0.6) (layer "F.Cu") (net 19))
 (segment (start 147.1593 98.552) (end 144.1833 101.528) (width 0.6) (layer "F.Cu") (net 19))
 (segment (start 143.6433 99.528) (end 139.68 99.528) (width 0.6) (layer "F.Cu") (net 20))
 (segment (start 147.1593 96.012) (end 143.6433 99.528) (width 0.6) (layer "F.Cu") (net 20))
 (segment (start 148.336 96.012) (end 147.1593 96.012) (width 0.6) (layer "F.Cu") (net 20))
 (segment (start 148.336 93.472) (end 147.1593 93.472) (width 0.6) (layer "F.Cu") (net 21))
 (segment (start 143.1033 97.528) (end 139.68 97.528) (width 0.6) (layer "F.Cu") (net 21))
 (segment (start 147.1593 93.472) (end 143.1033 97.528) (width 0.6) (layer "F.Cu") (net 21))
 (segment (start 147.1593 90.932) (end 142.5633 95.528) (width 0.6) (layer "F.Cu") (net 22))
 (segment (start 142.5633 95.528) (end 139.68 95.528) (width 0.6) (layer "F.Cu") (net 22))
 (segment (start 148.336 90.932) (end 147.1593 90.932) (width 0.6) (layer "F.Cu") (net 22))
 (segment (start 148.336 88.392) (end 146.3927 88.392) (width 0.6) (layer "F.Cu") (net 23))
 (segment (start 146.3927 88.392) (end 141.2567 93.528) (width 0.6) (layer "F.Cu") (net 23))
 (segment (start 139.68 93.528) (end 141.2567 93.528) (width 0.6) (layer "F.Cu") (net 23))
 (segment (start 149.86 114.651) (end 149.86 118.364) (width 0.8) (layer "F.Cu") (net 1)))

